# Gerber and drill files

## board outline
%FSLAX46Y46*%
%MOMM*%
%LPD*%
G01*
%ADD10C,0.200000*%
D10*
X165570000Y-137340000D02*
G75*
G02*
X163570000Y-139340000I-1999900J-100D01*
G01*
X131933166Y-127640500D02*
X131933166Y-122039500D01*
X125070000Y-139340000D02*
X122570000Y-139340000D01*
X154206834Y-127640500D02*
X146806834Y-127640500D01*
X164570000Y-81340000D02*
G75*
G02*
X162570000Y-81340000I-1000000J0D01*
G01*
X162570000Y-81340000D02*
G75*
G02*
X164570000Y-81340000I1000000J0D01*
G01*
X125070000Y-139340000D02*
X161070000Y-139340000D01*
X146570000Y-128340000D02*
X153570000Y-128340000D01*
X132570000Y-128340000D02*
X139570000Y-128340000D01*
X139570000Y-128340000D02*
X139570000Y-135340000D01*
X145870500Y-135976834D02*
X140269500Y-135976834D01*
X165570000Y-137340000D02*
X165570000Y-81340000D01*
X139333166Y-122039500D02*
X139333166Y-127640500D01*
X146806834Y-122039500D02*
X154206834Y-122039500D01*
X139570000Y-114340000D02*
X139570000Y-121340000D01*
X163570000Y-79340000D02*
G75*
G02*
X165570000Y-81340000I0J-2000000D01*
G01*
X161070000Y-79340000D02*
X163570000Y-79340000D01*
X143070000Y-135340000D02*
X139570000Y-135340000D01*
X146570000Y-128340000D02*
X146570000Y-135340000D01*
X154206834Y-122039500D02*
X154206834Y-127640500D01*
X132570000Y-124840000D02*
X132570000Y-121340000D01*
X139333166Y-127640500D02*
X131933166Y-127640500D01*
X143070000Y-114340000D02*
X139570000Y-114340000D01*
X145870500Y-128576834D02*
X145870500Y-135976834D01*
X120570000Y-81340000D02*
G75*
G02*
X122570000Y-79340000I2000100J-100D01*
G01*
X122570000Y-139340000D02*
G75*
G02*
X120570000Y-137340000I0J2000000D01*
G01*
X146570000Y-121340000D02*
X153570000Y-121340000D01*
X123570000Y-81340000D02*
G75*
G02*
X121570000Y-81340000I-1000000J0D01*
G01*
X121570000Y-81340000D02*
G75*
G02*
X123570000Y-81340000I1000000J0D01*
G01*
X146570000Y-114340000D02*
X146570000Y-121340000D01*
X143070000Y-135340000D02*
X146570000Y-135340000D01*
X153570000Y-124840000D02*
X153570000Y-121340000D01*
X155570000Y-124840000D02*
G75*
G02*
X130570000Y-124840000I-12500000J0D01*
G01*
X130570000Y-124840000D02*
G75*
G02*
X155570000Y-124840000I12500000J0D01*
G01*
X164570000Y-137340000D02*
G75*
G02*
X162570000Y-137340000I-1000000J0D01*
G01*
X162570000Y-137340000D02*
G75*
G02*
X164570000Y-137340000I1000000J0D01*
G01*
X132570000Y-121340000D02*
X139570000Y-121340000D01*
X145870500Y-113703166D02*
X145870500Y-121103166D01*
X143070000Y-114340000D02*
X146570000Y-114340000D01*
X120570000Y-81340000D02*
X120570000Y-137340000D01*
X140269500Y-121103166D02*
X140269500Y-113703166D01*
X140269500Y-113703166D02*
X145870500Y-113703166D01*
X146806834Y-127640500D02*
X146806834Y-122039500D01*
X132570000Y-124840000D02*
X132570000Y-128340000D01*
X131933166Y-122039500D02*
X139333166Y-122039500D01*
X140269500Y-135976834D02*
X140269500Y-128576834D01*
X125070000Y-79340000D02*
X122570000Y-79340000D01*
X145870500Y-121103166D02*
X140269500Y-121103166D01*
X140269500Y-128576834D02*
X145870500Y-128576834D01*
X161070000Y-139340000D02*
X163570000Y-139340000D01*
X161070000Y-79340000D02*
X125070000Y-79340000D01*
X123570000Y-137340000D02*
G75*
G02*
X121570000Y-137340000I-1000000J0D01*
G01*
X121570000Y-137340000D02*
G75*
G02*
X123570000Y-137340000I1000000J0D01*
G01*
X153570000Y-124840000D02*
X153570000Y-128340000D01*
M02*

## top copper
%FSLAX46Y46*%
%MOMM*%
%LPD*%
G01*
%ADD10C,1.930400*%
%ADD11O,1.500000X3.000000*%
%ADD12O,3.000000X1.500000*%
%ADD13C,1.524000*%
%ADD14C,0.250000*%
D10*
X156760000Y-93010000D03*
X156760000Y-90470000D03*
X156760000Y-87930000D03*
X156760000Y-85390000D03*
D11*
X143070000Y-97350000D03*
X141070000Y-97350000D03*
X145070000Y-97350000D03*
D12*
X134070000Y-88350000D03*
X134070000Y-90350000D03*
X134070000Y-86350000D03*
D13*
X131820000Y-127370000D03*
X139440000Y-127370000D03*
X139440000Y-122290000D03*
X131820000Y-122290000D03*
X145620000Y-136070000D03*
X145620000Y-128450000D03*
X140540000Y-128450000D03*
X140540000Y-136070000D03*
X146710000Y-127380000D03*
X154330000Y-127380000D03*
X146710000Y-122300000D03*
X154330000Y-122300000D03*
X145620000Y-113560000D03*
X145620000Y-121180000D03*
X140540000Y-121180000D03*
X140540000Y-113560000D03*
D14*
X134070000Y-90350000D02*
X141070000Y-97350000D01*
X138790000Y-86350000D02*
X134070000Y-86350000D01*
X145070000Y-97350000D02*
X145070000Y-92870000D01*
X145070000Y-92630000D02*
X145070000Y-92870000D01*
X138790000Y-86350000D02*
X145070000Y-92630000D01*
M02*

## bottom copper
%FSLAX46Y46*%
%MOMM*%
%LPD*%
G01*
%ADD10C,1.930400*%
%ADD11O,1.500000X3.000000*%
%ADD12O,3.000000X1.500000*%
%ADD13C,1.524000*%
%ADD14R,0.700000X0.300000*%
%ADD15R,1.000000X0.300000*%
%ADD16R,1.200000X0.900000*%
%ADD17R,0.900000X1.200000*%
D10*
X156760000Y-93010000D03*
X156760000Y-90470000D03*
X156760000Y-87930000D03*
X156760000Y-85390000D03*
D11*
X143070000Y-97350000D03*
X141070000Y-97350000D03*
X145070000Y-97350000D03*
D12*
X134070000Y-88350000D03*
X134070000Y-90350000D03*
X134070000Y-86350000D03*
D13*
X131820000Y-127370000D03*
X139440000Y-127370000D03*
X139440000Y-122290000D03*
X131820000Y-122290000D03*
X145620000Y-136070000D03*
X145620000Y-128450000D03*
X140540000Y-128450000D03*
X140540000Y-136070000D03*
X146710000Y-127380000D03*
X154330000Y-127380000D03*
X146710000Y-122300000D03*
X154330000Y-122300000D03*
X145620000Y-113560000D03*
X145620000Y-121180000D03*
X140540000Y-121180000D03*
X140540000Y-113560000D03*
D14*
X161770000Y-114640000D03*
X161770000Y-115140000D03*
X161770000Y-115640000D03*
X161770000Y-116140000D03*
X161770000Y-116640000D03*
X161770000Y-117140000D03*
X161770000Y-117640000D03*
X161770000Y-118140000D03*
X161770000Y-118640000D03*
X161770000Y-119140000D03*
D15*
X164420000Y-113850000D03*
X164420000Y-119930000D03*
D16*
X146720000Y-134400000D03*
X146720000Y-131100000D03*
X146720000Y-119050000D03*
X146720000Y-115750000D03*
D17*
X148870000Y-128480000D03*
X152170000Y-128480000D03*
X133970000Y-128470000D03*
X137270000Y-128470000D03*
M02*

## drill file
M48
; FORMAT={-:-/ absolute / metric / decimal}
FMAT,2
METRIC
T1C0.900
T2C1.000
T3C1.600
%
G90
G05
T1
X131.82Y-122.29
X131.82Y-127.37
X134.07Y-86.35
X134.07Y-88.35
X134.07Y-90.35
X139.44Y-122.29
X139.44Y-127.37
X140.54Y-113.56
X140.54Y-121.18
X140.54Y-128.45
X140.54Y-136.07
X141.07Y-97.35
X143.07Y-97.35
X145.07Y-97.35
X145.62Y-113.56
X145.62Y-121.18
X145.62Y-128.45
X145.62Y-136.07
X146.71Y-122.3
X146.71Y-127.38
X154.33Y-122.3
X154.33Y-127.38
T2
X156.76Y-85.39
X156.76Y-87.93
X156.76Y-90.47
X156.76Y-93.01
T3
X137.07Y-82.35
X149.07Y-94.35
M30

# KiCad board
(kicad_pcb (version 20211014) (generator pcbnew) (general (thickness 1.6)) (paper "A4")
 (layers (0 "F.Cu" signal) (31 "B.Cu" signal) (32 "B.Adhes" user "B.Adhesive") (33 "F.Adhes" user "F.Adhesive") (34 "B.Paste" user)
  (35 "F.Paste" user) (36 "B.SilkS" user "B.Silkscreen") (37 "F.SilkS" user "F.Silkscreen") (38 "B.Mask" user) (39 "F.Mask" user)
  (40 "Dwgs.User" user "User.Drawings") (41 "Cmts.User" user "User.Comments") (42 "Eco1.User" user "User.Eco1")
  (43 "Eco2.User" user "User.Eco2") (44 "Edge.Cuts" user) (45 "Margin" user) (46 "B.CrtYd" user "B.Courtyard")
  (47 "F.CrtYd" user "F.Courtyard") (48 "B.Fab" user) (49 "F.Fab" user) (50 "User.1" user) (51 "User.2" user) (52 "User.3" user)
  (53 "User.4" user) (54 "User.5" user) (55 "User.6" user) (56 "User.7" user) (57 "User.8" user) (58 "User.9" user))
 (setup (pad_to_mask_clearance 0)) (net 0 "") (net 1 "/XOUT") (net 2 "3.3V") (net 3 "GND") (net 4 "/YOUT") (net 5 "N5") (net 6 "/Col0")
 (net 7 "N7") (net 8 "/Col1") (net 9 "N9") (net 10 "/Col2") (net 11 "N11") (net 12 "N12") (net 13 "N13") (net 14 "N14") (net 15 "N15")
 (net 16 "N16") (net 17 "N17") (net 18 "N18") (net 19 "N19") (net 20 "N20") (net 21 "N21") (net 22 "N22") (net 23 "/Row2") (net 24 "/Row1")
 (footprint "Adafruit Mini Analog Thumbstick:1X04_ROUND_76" (layer "F.Cu") (at 156.76 89.2 90)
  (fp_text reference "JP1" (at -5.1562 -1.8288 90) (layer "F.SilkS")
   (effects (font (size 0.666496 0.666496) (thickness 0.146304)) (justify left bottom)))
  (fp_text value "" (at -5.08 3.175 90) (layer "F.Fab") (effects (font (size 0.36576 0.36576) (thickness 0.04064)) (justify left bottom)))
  (pad "1" thru_hole circle (at -3.81 0 180) (size 1.9304 1.9304) (drill 1) (layers *.Cu *.Mask) (solder_mask_margin 0.0508))
  (pad "2" thru_hole circle (at -1.27 0 180) (size 1.9304 1.9304) (drill 1) (layers *.Cu *.Mask) (solder_mask_margin 0.0508))
  (pad "3" thru_hole circle (at 1.27 0 180) (size 1.9304 1.9304) (drill 1) (layers *.Cu *.Mask) (solder_mask_margin 0.0508))
  (pad "4" thru_hole circle (at 3.81 0 180) (size 1.9304 1.9304) (drill 1) (layers *.Cu *.Mask) (solder_mask_margin 0.0508)))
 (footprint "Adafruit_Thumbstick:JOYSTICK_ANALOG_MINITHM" (layer "F.Cu") (at 143.07 88.35 180)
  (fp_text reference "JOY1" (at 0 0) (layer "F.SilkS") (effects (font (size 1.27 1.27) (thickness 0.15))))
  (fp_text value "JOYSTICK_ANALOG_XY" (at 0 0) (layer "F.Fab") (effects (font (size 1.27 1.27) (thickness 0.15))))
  (pad "" np_thru_hole circle (at -6 -6 180) (size 1.6 1.6) (drill 1.6) (layers *.Cu *.Mask))
  (pad "" np_thru_hole circle (at 6 6 180) (size 1.6 1.6) (drill 1.6) (layers *.Cu *.Mask))
  (pad "X" thru_hole oval (at 0 -9 270) (size 3 1.5) (drill 0.9) (layers *.Cu *.Mask) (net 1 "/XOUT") (solder_mask_margin 0.0508))
  (pad "X+" thru_hole oval (at 2 -9 270) (size 3 1.5) (drill 0.9) (layers *.Cu *.Mask) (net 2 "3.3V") (solder_mask_margin 0.0508))
  (pad "X-" thru_hole oval (at -2 -9 270) (size 3 1.5) (drill 0.9) (layers *.Cu *.Mask) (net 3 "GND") (solder_mask_margin 0.0508))
  (pad "Y" thru_hole oval (at 9 0 180) (size 3 1.5) (drill 0.9) (layers *.Cu *.Mask) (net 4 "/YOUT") (solder_mask_margin 0.0508))
  (pad "Y+" thru_hole oval (at 9 -2 180) (size 3 1.5) (drill 0.9) (layers *.Cu *.Mask) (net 2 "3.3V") (solder_mask_margin 0.0508))
  (pad "Y-" thru_hole oval (at 9 2 180) (size 3 1.5) (drill 0.9) (layers *.Cu *.Mask) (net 3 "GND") (solder_mask_margin 0.0508)))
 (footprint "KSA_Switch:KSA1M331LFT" (layer "F.Cu") (at 135.63 124.83 90)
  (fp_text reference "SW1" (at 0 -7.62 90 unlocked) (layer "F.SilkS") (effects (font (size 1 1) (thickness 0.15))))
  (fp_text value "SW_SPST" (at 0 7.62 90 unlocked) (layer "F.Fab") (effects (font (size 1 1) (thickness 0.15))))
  (pad "1" thru_hole circle (at -2.54 -3.81 90) (size 1.524 1.524) (drill 0.9) (layers *.Cu *.Mask) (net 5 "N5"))
  (pad "1" thru_hole circle (at -2.54 3.81 90) (size 1.524 1.524) (drill 0.9) (layers *.Cu *.Mask) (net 5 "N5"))
  (pad "2" thru_hole circle (at 2.54 3.81 90) (size 1.524 1.524) (drill 0.9) (layers *.Cu *.Mask) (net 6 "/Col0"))
  (pad "2" thru_hole circle (at 2.54 -3.81 90) (size 1.524 1.524) (drill 0.9) (layers *.Cu *.Mask) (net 6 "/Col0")))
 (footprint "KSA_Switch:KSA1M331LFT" (layer "F.Cu") (at 143.08 132.26 180)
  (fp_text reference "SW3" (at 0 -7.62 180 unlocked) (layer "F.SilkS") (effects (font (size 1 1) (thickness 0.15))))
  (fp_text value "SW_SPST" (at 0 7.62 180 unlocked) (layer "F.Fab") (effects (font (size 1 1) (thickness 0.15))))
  (pad "1" thru_hole circle (at -2.54 -3.81 180) (size 1.524 1.524) (drill 0.9) (layers *.Cu *.Mask) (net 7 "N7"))
  (pad "1" thru_hole circle (at -2.54 3.81 180) (size 1.524 1.524) (drill 0.9) (layers *.Cu *.Mask) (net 7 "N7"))
  (pad "2" thru_hole circle (at 2.54 3.81 180) (size 1.524 1.524) (drill 0.9) (layers *.Cu *.Mask) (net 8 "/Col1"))
  (pad "2" thru_hole circle (at 2.54 -3.81 180) (size 1.524 1.524) (drill 0.9) (layers *.Cu *.Mask) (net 8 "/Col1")))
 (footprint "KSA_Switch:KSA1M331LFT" (layer "F.Cu") (at 150.52 124.84 90)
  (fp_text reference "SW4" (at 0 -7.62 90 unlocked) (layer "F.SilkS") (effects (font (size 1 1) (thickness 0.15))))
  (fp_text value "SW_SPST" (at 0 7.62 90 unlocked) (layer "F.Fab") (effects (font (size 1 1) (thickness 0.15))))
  (pad "1" thru_hole circle (at -2.54 -3.81 90) (size 1.524 1.524) (drill 0.9) (layers *.Cu *.Mask) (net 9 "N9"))
  (pad "1" thru_hole circle (at -2.54 3.81 90) (size 1.524 1.524) (drill 0.9) (layers *.Cu *.Mask) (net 9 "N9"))
  (pad "2" thru_hole circle (at 2.54 -3.81 90) (size 1.524 1.524) (drill 0.9) (layers *.Cu *.Mask) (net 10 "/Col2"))
  (pad "2" thru_hole circle (at 2.54 3.81 90) (size 1.524 1.524) (drill 0.9) (layers *.Cu *.Mask) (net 10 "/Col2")))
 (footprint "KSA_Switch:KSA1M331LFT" (layer "F.Cu") (at 143.08 117.37 180)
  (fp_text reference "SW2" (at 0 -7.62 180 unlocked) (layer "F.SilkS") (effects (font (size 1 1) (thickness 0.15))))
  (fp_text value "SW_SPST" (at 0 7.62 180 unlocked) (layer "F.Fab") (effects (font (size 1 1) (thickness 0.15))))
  (pad "1" thru_hole circle (at -2.54 3.81 180) (size 1.524 1.524) (drill 0.9) (layers *.Cu *.Mask) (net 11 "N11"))
  (pad "1" thru_hole circle (at -2.54 -3.81 180) (size 1.524 1.524) (drill 0.9) (layers *.Cu *.Mask) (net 11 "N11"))
  (pad "2" thru_hole circle (at 2.54 -3.81 180) (size 1.524 1.524) (drill 0.9) (layers *.Cu *.Mask) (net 8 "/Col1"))
  (pad "2" thru_hole circle (at 2.54 3.81 180) (size 1.524 1.524) (drill 0.9) (layers *.Cu *.Mask) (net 8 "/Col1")))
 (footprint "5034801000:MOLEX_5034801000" (layer "B.Cu") (at 161.77 116.89 -90)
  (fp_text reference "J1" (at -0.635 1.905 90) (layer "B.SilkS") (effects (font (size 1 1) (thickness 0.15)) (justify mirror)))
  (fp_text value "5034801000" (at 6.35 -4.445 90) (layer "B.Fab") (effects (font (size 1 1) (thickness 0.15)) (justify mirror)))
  (pad "1" smd rect locked (at -2.25 0 270) (size 0.3 0.7) (layers "B.Cu" "B.Paste" "B.Mask") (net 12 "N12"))
  (pad "2" smd rect locked (at -1.75 0 270) (size 0.3 0.7) (layers "B.Cu" "B.Paste" "B.Mask") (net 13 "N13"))
  (pad "3" smd rect locked (at -1.25 0 270) (size 0.3 0.7) (layers "B.Cu" "B.Paste" "B.Mask") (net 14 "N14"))
  (pad "4" smd rect locked (at -0.75 0 270) (size 0.3 0.7) (layers "B.Cu" "B.Paste" "B.Mask") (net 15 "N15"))
  (pad "5" smd rect locked (at -0.25 0 270) (size 0.3 0.7) (layers "B.Cu" "B.Paste" "B.Mask") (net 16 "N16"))
  (pad "6" smd rect locked (at 0.25 0 270) (size 0.3 0.7) (layers "B.Cu" "B.Paste" "B.Mask") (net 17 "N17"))
  (pad "7" smd rect locked (at 0.75 0 270) (size 0.3 0.7) (layers "B.Cu" "B.Paste" "B.Mask") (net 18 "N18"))
  (pad "8" smd rect locked (at 1.25 0 270) (size 0.3 0.7) (layers "B.Cu" "B.Paste" "B.Mask") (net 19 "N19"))
  (pad "9" smd rect locked (at 1.75 0 270) (size 0.3 0.7) (layers "B.Cu" "B.Paste" "B.Mask") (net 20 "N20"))
  (pad "10" smd rect locked (at 2.25 0 270) (size 0.3 0.7) (layers "B.Cu" "B.Paste" "B.Mask") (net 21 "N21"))
  (pad "S1" smd rect locked (at -3.04 -2.65 270) (size 0.3 1) (layers "B.Cu" "B.Paste" "B.Mask") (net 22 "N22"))
  (pad "S2" smd rect locked (at 3.04 -2.65 270) (size 0.3 1) (layers "B.Cu" "B.Paste" "B.Mask") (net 22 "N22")))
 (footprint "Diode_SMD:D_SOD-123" (layer "B.Cu") (at 146.72 132.75 90)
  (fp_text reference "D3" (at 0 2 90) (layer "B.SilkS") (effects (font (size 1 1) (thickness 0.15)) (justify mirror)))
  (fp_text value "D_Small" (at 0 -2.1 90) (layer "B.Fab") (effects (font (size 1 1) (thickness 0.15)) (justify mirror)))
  (pad "1" smd rect (at -1.65 0 90) (size 0.9 1.2) (layers "B.Cu" "B.Paste" "B.Mask") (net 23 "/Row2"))
  (pad "2" smd rect (at 1.65 0 90) (size 0.9 1.2) (layers "B.Cu" "B.Paste" "B.Mask") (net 7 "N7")))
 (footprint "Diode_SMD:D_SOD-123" (layer "B.Cu") (at 146.72 117.4 90)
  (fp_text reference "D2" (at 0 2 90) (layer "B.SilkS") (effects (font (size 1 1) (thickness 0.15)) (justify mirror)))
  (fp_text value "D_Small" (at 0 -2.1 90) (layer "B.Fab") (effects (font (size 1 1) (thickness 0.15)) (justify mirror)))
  (pad "1" smd rect (at -1.65 0 90) (size 0.9 1.2) (layers "B.Cu" "B.Paste" "B.Mask") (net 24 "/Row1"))
  (pad "2" smd rect (at 1.65 0 90) (size 0.9 1.2) (layers "B.Cu" "B.Paste" "B.Mask") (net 11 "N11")))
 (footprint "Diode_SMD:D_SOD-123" (layer "B.Cu") (at 150.52 128.48)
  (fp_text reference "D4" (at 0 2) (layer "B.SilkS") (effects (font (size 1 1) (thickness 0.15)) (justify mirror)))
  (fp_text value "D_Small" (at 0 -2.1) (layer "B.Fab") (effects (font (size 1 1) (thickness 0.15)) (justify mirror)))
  (pad "1" smd rect (at -1.65 0) (size 0.9 1.2) (layers "B.Cu" "B.Paste" "B.Mask") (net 23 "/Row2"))
  (pad "2" smd rect (at 1.65 0) (size 0.9 1.2) (layers "B.Cu" "B.Paste" "B.Mask") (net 9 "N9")))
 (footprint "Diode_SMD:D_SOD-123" (layer "B.Cu") (at 135.62 128.47)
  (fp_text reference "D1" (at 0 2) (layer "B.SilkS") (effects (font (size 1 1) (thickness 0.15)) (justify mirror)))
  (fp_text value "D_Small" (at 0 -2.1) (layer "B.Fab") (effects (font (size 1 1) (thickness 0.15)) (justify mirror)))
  (pad "1" smd rect (at -1.65 0) (size 0.9 1.2) (layers "B.Cu" "B.Paste" "B.Mask") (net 23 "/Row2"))
  (pad "2" smd rect (at 1.65 0) (size 0.9 1.2) (layers "B.Cu" "B.Paste" "B.Mask") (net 5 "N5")))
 (gr_arc (start 165.57 137.34) (mid 164.984227 138.754245) (end 163.57 139.34) (layer "Edge.Cuts") (width 0.2))
 (gr_line (start 131.933166 127.6405) (end 131.933166 122.0395) (layer "Edge.Cuts") (width 0.2))
 (gr_line (start 125.07 139.34) (end 122.57 139.34) (layer "Edge.Cuts") (width 0.2))
 (gr_line (start 154.206834 127.6405) (end 146.806834 127.6405) (layer "Edge.Cuts") (width 0.2))
 (gr_circle (center 163.57 81.34) (end 164.57 81.34) (layer "Edge.Cuts") (width 0.2) (fill none))
 (gr_line (start 125.07 139.34) (end 161.07 139.34) (layer "Edge.Cuts") (width 0.2))
 (gr_line (start 146.57 128.34) (end 153.57 128.34) (layer "Edge.Cuts") (width 0.2))
 (gr_line (start 132.57 128.34) (end 139.57 128.34) (layer "Edge.Cuts") (width 0.2))
 (gr_line (start 139.57 128.34) (end 139.57 135.34) (layer "Edge.Cuts") (width 0.2))
 (gr_line (start 145.8705 135.976834) (end 140.2695 135.976834) (layer "Edge.Cuts") (width 0.2))
 (gr_line (start 165.57 137.34) (end 165.57 81.34) (layer "Edge.Cuts") (width 0.2))
 (gr_line (start 139.333166 122.0395) (end 139.333166 127.6405) (layer "Edge.Cuts") (width 0.2))
 (gr_line (start 146.806834 122.0395) (end 154.206834 122.0395) (layer "Edge.Cuts") (width 0.2))
 (gr_line (start 139.57 114.34) (end 139.57 121.34) (layer "Edge.Cuts") (width 0.2))
 (gr_arc (start 163.57 79.34) (mid 164.98421 79.925793) (end 165.57 81.34) (layer "Edge.Cuts") (width 0.2))
 (gr_line (start 161.07 79.34) (end 163.57 79.34) (layer "Edge.Cuts") (width 0.2))
 (gr_line (start 143.07 135.34) (end 139.57 135.34) (layer "Edge.Cuts") (width 0.2))
 (gr_line (start 146.57 128.34) (end 146.57 135.34) (layer "Edge.Cuts") (width 0.2))
 (gr_line (start 154.206834 122.0395) (end 154.206834 127.6405) (layer "Edge.Cuts") (width 0.2))
 (gr_line (start 132.57 124.84) (end 132.57 121.34) (layer "Edge.Cuts") (width 0.2))
 (gr_line (start 139.333166 127.6405) (end 131.933166 127.6405) (layer "Edge.Cuts") (width 0.2))
 (gr_line (start 143.07 114.34) (end 139.57 114.34) (layer "Edge.Cuts") (width 0.2))
 (gr_line (start 145.8705 128.576834) (end 145.8705 135.976834) (layer "Edge.Cuts") (width 0.2))
 (gr_arc (start 120.57 81.34) (mid 121.1558 79.925818) (end 122.57 79.34) (layer "Edge.Cuts") (width 0.2))
 (gr_arc (start 122.57 139.34) (mid 121.155783 138.75422) (end 120.57 137.34) (layer "Edge.Cuts") (width 0.2))
 (gr_line (start 146.57 121.34) (end 153.57 121.34) (layer "Edge.Cuts") (width 0.2))
 (gr_circle (center 122.57 81.34) (end 123.57 81.34) (layer "Edge.Cuts") (width 0.2) (fill none))
 (gr_line (start 146.57 114.34) (end 146.57 121.34) (layer "Edge.Cuts") (width 0.2))
 (gr_line (start 143.07 135.34) (end 146.57 135.34) (layer "Edge.Cuts") (width 0.2))
 (gr_line (start 153.57 124.84) (end 153.57 121.34) (layer "Edge.Cuts") (width 0.2))
 (gr_circle (center 143.07 124.84) (end 155.57 124.84) (layer "Edge.Cuts") (width 0.2) (fill none))
 (gr_circle (center 163.57 137.34) (end 164.57 137.34) (layer "Edge.Cuts") (width 0.2) (fill none))
 (gr_line (start 132.57 121.34) (end 139.57 121.34) (layer "Edge.Cuts") (width 0.2))
 (gr_line (start 145.8705 113.703166) (end 145.8705 121.103166) (layer "Edge.Cuts") (width 0.2))
 (gr_line (start 143.07 114.34) (end 146.57 114.34) (layer "Edge.Cuts") (width 0.2))
 (gr_line (start 120.57 81.34) (end 120.57 137.34) (layer "Edge.Cuts") (width 0.2))
 (gr_line (start 140.2695 121.103166) (end 140.2695 113.703166) (layer "Edge.Cuts") (width 0.2))
 (gr_line (start 140.2695 113.703166) (end 145.8705 113.703166) (layer "Edge.Cuts") (width 0.2))
 (gr_line (start 146.806834 127.6405) (end 146.806834 122.0395) (layer "Edge.Cuts") (width 0.2))
 (gr_line (start 132.57 124.84) (end 132.57 128.34) (layer "Edge.Cuts") (width 0.2))
 (gr_line (start 131.933166 122.0395) (end 139.333166 122.0395) (layer "Edge.Cuts") (width 0.2))
 (gr_line (start 140.2695 135.976834) (end 140.2695 128.576834) (layer "Edge.Cuts") (width 0.2))
 (gr_line (start 125.07 79.34) (end 122.57 79.34) (layer "Edge.Cuts") (width 0.2))
 (gr_line (start 145.8705 121.103166) (end 140.2695 121.103166) (layer "Edge.Cuts") (width 0.2))
 (gr_line (start 140.2695 128.576834) (end 145.8705 128.576834) (layer "Edge.Cuts") (width 0.2))
 (gr_line (start 161.07 139.34) (end 163.57 139.34) (layer "Edge.Cuts") (width 0.2))
 (gr_line (start 161.07 79.34) (end 125.07 79.34) (layer "Edge.Cuts") (width 0.2))
 (gr_circle (center 122.57 137.34) (end 123.57 137.34) (layer "Edge.Cuts") (width 0.2) (fill none))
 (gr_line (start 153.57 124.84) (end 153.57 128.34) (layer "Edge.Cuts") (width 0.2))
 (segment (start 134.07 90.35) (end 141.07 97.35) (width 0.25) (layer "F.Cu") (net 2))
 (segment (start 138.79 86.35) (end 134.07 86.35) (width 0.25) (layer "F.Cu") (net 3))
 (segment (start 145.07 97.35) (end 145.07 92.87) (width 0.25) (layer "F.Cu") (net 3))
 (segment (start 145.07 92.63) (end 145.07 92.87) (width 0.25) (layer "F.Cu") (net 3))
 (segment (start 138.79 86.35) (end 145.07 92.63) (width 0.25) (layer "F.Cu") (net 3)))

